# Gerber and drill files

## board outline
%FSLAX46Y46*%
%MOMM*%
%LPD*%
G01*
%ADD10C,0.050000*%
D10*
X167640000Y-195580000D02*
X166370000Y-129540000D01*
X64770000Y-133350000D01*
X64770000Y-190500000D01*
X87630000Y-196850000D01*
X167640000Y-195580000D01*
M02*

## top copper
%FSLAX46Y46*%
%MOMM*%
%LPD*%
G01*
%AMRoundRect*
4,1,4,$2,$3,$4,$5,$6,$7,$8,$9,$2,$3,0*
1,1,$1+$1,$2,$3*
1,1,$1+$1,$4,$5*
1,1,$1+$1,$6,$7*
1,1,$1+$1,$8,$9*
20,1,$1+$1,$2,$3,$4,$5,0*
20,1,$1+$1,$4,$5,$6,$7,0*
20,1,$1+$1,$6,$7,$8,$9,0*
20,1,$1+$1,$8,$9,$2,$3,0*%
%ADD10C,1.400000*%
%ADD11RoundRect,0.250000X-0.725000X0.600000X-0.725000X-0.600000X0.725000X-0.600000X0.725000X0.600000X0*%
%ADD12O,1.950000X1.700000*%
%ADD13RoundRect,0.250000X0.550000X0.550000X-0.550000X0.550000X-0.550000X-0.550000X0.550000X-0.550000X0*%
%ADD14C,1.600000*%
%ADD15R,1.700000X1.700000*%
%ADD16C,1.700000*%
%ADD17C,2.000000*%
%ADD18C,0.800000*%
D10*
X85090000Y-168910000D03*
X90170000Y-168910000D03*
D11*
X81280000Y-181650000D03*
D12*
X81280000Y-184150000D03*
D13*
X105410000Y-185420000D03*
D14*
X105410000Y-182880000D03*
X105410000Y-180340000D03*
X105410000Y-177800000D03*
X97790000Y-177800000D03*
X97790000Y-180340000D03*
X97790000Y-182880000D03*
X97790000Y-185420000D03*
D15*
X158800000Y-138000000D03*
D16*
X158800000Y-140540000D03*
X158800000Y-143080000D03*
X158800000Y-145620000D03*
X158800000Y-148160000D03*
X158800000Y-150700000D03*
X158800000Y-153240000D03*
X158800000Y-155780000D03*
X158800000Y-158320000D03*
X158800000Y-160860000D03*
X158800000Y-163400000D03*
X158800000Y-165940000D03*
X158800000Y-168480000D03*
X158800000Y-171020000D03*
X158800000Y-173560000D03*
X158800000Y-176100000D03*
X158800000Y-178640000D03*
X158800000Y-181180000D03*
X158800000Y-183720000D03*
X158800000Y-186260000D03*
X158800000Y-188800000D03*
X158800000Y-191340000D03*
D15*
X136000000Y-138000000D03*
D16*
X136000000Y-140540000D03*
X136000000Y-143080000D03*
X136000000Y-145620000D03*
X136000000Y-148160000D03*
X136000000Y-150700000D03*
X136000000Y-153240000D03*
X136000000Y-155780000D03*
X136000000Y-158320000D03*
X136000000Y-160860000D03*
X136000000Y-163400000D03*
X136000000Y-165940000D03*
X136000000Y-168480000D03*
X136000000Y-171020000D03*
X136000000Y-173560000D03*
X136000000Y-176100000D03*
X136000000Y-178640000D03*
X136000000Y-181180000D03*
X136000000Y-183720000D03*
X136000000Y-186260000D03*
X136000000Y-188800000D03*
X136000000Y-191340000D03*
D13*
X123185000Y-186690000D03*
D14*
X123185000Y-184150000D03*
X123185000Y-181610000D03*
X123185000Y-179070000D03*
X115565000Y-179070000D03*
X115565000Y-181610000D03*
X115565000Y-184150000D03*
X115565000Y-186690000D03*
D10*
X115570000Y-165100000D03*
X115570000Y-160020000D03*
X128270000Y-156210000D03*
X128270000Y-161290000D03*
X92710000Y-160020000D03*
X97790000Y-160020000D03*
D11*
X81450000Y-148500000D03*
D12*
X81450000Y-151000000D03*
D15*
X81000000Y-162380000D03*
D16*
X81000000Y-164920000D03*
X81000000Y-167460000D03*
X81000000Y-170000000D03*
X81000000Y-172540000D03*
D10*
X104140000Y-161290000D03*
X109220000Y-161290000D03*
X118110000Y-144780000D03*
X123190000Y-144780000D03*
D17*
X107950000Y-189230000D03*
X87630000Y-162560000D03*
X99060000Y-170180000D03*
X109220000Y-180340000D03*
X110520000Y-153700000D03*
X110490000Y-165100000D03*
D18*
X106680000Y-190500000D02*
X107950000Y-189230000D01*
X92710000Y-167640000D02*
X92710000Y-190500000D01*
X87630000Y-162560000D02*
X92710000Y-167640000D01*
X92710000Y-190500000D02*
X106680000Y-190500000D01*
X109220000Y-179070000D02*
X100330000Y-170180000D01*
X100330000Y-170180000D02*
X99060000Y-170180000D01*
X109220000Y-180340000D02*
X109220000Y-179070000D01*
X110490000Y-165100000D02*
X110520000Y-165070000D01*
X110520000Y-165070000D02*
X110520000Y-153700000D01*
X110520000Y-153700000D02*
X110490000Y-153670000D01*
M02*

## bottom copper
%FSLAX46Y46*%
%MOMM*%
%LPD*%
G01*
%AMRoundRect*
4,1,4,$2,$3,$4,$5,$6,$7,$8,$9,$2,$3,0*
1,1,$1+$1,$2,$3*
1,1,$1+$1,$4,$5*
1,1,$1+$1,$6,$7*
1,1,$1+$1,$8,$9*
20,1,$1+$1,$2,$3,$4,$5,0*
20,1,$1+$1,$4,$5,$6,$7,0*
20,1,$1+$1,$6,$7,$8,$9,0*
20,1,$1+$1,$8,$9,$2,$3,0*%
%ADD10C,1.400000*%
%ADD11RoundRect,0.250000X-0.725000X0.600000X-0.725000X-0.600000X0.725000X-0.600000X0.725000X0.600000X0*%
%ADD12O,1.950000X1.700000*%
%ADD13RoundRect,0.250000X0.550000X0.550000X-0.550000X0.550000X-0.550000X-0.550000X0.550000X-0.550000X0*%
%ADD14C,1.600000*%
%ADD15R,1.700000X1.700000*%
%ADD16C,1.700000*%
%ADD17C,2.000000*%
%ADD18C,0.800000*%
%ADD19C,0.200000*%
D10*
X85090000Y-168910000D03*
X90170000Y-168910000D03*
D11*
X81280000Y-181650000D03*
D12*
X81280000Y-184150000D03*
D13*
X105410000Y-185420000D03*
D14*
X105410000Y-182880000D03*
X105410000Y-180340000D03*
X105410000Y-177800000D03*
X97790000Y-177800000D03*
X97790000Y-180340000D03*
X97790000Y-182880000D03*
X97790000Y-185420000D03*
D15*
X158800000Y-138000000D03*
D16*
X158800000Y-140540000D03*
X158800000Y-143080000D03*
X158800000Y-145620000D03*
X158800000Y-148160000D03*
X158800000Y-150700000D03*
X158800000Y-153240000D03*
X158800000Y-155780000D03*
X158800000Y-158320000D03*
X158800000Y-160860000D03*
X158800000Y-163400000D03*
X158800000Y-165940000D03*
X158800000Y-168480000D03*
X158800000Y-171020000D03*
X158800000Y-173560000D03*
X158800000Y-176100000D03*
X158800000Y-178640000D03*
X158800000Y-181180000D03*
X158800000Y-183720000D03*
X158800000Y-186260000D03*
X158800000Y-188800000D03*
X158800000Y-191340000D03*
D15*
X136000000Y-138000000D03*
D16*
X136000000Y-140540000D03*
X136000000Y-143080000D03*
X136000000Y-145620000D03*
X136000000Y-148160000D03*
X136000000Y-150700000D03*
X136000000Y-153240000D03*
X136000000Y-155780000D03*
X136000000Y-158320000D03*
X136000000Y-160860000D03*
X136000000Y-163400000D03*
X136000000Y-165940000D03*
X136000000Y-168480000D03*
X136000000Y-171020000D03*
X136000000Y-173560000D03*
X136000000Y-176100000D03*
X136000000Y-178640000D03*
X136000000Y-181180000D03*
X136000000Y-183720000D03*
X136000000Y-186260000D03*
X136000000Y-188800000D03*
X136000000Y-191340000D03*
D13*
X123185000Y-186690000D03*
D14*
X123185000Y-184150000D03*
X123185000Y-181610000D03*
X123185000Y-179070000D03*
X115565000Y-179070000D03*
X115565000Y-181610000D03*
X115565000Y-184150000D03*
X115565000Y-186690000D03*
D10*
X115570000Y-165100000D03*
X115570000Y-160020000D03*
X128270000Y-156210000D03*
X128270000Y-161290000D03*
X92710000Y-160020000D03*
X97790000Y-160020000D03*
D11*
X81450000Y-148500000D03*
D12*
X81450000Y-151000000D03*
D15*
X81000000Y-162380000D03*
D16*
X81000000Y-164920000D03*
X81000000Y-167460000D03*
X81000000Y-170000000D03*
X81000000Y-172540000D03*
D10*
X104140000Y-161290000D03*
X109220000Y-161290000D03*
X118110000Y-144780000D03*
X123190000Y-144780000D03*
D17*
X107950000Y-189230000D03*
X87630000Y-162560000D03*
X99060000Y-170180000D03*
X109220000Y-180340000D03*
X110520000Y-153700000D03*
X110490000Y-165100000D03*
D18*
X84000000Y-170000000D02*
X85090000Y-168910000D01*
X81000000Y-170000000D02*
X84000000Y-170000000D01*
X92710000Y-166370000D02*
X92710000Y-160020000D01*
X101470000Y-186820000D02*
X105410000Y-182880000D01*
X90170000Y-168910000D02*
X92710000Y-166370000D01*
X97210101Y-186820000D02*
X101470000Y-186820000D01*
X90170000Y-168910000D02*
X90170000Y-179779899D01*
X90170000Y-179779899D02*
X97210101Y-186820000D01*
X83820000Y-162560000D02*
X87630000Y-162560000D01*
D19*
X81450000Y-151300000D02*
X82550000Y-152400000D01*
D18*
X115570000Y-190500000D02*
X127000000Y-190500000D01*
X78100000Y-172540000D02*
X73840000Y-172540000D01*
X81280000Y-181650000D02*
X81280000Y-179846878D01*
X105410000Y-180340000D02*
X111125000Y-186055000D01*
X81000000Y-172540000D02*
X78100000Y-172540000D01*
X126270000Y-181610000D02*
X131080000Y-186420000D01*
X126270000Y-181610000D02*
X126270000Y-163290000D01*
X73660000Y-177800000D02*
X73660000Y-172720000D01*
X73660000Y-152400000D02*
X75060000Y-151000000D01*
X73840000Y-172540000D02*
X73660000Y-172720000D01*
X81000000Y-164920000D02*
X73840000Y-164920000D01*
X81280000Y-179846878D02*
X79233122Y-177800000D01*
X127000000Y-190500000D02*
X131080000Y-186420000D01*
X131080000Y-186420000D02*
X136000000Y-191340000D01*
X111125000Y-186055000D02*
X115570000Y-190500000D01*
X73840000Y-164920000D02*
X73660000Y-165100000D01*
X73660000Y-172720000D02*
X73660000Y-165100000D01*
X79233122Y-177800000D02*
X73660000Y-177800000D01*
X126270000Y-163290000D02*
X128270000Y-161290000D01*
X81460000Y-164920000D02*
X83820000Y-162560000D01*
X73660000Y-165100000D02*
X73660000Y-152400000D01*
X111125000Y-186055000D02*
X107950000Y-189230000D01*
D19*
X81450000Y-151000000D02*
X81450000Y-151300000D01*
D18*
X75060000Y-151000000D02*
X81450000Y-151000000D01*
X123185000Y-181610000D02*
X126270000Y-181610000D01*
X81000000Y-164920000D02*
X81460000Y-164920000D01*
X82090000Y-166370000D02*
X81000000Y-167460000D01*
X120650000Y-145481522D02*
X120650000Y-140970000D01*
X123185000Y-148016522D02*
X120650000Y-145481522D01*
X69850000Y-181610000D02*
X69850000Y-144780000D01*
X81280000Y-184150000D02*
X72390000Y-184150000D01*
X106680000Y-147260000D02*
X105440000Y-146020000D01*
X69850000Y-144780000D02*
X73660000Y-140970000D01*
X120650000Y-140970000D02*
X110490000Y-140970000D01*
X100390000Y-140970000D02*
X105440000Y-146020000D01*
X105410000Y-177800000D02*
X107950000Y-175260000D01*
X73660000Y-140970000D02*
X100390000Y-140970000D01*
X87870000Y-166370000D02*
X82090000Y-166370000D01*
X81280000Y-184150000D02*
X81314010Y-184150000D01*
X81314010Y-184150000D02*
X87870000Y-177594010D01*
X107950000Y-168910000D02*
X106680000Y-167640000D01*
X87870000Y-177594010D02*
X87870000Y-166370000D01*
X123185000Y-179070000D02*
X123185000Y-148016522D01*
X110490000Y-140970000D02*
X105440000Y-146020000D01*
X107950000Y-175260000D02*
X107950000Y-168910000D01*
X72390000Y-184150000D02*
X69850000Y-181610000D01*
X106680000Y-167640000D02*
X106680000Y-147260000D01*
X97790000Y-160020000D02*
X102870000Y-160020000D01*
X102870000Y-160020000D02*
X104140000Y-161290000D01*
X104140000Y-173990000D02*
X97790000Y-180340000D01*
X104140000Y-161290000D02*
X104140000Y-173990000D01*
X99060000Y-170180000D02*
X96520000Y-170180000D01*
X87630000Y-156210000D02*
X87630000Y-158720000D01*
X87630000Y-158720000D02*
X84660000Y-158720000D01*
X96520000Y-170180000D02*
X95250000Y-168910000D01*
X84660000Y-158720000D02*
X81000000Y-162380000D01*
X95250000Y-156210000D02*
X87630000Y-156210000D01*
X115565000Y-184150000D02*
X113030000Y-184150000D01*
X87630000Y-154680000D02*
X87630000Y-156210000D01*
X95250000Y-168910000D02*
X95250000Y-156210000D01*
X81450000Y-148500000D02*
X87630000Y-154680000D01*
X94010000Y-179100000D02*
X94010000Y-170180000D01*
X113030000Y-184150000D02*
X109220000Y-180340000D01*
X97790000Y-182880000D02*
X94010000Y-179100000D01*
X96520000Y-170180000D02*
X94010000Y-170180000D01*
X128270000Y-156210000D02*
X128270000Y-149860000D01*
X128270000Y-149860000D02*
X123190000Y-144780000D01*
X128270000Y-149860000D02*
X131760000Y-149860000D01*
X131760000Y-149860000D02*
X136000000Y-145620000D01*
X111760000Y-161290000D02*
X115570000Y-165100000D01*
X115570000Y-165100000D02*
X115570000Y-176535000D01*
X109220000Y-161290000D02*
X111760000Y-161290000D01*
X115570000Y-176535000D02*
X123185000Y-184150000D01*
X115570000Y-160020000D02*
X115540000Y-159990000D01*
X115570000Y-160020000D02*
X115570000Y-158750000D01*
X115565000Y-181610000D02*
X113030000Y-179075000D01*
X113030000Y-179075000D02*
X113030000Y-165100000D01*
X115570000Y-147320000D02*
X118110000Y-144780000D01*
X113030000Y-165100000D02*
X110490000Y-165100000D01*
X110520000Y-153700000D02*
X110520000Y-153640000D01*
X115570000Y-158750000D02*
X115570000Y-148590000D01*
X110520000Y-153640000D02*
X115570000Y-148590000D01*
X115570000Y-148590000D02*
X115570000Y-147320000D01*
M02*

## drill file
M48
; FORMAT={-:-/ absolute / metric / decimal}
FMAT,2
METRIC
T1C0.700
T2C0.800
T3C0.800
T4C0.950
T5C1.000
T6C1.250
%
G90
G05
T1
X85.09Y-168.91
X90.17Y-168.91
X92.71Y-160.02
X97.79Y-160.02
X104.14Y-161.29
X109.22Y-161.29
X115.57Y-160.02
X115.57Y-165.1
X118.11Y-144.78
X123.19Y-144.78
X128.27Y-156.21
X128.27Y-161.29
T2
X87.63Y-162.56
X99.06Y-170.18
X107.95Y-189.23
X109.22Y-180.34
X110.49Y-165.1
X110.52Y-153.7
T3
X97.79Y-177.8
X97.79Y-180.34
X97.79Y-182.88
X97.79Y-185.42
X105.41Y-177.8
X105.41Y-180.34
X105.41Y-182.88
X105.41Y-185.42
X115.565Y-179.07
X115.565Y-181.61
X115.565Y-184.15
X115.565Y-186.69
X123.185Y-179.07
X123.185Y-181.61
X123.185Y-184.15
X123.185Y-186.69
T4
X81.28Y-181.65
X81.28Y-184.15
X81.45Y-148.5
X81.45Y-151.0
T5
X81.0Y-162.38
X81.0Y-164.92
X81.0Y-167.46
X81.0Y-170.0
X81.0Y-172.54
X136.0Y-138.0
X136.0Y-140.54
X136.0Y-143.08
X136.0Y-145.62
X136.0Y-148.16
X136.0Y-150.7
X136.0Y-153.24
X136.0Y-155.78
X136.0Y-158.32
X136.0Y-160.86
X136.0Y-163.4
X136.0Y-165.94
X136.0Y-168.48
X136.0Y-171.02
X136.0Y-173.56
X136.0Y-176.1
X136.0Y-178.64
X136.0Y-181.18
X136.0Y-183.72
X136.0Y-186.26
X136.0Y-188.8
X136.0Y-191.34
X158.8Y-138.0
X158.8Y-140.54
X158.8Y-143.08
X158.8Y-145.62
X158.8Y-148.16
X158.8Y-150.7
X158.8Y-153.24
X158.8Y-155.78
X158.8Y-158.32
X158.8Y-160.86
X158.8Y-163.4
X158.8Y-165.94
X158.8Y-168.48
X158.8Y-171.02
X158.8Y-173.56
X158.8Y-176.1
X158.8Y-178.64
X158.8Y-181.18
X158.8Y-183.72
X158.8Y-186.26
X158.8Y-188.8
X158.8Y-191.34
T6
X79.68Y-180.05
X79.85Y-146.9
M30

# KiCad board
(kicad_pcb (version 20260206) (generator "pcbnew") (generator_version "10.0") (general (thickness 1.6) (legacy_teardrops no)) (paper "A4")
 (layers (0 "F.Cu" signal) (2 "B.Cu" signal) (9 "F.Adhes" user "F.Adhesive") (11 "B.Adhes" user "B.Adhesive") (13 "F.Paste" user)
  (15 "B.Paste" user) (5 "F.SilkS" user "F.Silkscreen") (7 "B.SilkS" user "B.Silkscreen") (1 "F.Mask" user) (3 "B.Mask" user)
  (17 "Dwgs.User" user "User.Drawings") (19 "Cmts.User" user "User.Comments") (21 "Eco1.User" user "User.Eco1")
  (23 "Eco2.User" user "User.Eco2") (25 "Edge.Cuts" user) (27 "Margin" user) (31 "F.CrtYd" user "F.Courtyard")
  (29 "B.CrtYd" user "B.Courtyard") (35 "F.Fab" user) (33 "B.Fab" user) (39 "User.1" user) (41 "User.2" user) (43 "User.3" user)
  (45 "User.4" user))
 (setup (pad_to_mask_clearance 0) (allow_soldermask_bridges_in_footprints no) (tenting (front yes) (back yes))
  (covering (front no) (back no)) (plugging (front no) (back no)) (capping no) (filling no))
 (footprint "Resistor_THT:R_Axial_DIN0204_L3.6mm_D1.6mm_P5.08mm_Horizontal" (layer "F.Cu") (at 85.09 168.91)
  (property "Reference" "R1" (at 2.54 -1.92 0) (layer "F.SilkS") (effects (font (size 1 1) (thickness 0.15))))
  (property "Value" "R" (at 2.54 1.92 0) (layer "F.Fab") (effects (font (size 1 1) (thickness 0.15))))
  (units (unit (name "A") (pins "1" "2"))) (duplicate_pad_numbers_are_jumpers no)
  (pad "1" thru_hole circle (at 0 0) (size 1.4 1.4) (drill 0.7) (layers "*.Cu" "*.Mask") (remove_unused_layers no) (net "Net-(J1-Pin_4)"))
  (pad "2" thru_hole circle (at 5.08 0) (size 1.4 1.4) (drill 0.7) (layers "*.Cu" "*.Mask") (remove_unused_layers no) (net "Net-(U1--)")))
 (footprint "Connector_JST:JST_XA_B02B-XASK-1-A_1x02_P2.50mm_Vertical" (layer "F.Cu") (at 81.28 181.65 -90)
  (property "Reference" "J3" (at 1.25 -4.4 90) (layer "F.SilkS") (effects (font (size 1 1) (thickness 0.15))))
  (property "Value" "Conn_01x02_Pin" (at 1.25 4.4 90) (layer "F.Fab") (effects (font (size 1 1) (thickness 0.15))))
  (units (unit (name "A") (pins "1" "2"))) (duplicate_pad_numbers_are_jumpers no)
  (pad "" np_thru_hole circle (at -1.6 1.6 270) (size 1.25 1.25) (drill 1.25) (layers "*.Cu" "*.Mask"))
  (pad "1" thru_hole roundrect (at 0 0 270) (size 1.7 1.95) (drill 0.95) (layers "*.Cu" "*.Mask") (remove_unused_layers no)
   (roundrect_rratio 0.147059) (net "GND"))
  (pad "2" thru_hole oval (at 2.5 0 270) (size 1.7 1.95) (drill 0.95) (layers "*.Cu" "*.Mask") (remove_unused_layers no) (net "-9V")))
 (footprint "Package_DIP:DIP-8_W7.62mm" (layer "F.Cu") (at 105.41 185.42 180)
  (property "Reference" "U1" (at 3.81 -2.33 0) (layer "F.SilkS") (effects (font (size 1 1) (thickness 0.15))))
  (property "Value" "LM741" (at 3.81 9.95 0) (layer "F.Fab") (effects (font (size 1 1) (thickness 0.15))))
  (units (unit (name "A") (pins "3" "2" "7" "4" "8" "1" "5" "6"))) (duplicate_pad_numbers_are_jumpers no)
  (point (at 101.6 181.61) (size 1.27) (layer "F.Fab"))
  (pad "1" thru_hole roundrect (at 0 0 180) (size 1.6 1.6) (drill 0.8) (layers "*.Cu" "*.Mask") (remove_unused_layers no)
   (roundrect_rratio 0.15625) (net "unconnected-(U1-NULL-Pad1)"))
  (pad "2" thru_hole circle (at 0 2.54 180) (size 1.6 1.6) (drill 0.8) (layers "*.Cu" "*.Mask") (remove_unused_layers no) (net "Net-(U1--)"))
  (pad "3" thru_hole circle (at 0 5.08 180) (size 1.6 1.6) (drill 0.8) (layers "*.Cu" "*.Mask") (remove_unused_layers no) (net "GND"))
  (pad "4" thru_hole circle (at 0 7.62 180) (size 1.6 1.6) (drill 0.8) (layers "*.Cu" "*.Mask") (remove_unused_layers no) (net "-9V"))
  (pad "5" thru_hole circle (at 7.62 7.62 180) (size 1.6 1.6) (drill 0.8) (layers "*.Cu" "*.Mask") (remove_unused_layers no)
   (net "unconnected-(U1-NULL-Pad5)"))
  (pad "6" thru_hole circle (at 7.62 5.08 180) (size 1.6 1.6) (drill 0.8) (layers "*.Cu" "*.Mask") (remove_unused_layers no)
   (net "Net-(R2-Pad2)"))
  (pad "7" thru_hole circle (at 7.62 2.54 180) (size 1.6 1.6) (drill 0.8) (layers "*.Cu" "*.Mask") (remove_unused_layers no) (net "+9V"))
  (pad "8" thru_hole circle (at 7.62 0 180) (size 1.6 1.6) (drill 0.8) (layers "*.Cu" "*.Mask") (remove_unused_layers no)
   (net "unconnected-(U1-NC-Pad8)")))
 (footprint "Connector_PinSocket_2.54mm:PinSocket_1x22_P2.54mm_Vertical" (layer "F.Cu") (at 158.8 138)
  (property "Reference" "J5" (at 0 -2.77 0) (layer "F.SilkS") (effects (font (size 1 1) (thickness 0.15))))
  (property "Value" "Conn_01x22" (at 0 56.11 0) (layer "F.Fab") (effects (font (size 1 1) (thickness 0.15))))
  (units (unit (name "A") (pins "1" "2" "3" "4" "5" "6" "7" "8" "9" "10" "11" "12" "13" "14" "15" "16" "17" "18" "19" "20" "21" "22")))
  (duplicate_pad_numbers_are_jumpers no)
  (pad "1" thru_hole rect (at 0 0) (size 1.7 1.7) (drill 1) (layers "*.Cu" "*.Mask") (remove_unused_layers no)
   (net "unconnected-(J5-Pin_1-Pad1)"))
  (pad "2" thru_hole circle (at 0 2.54) (size 1.7 1.7) (drill 1) (layers "*.Cu" "*.Mask") (remove_unused_layers no)
   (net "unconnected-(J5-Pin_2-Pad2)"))
  (pad "3" thru_hole circle (at 0 5.08) (size 1.7 1.7) (drill 1) (layers "*.Cu" "*.Mask") (remove_unused_layers no)
   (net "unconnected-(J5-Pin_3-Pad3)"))
  (pad "4" thru_hole circle (at 0 7.62) (size 1.7 1.7) (drill 1) (layers "*.Cu" "*.Mask") (remove_unused_layers no)
   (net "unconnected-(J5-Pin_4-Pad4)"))
  (pad "5" thru_hole circle (at 0 10.16) (size 1.7 1.7) (drill 1) (layers "*.Cu" "*.Mask") (remove_unused_layers no)
   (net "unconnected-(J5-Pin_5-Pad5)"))
  (pad "6" thru_hole circle (at 0 12.7) (size 1.7 1.7) (drill 1) (layers "*.Cu" "*.Mask") (remove_unused_layers no)
   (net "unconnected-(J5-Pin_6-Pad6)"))
  (pad "7" thru_hole circle (at 0 15.24) (size 1.7 1.7) (drill 1) (layers "*.Cu" "*.Mask") (remove_unused_layers no)
   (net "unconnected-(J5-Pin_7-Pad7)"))
  (pad "8" thru_hole circle (at 0 17.78) (size 1.7 1.7) (drill 1) (layers "*.Cu" "*.Mask") (remove_unused_layers no)
   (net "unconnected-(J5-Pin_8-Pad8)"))
  (pad "9" thru_hole circle (at 0 20.32) (size 1.7 1.7) (drill 1) (layers "*.Cu" "*.Mask") (remove_unused_layers no)
   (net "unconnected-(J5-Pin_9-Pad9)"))
  (pad "10" thru_hole circle (at 0 22.86) (size 1.7 1.7) (drill 1) (layers "*.Cu" "*.Mask") (remove_unused_layers no)
   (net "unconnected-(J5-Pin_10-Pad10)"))
  (pad "11" thru_hole circle (at 0 25.4) (size 1.7 1.7) (drill 1) (layers "*.Cu" "*.Mask") (remove_unused_layers no)
   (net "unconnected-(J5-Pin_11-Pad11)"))
  (pad "12" thru_hole circle (at 0 27.94) (size 1.7 1.7) (drill 1) (layers "*.Cu" "*.Mask") (remove_unused_layers no)
   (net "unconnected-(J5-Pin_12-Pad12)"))
  (pad "13" thru_hole circle (at 0 30.48) (size 1.7 1.7) (drill 1) (layers "*.Cu" "*.Mask") (remove_unused_layers no)
   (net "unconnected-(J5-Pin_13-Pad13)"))
  (pad "14" thru_hole circle (at 0 33.02) (size 1.7 1.7) (drill 1) (layers "*.Cu" "*.Mask") (remove_unused_layers no)
   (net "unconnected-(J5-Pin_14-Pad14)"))
  (pad "15" thru_hole circle (at 0 35.56) (size 1.7 1.7) (drill 1) (layers "*.Cu" "*.Mask") (remove_unused_layers no)
   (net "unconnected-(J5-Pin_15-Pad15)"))
  (pad "16" thru_hole circle (at 0 38.1) (size 1.7 1.7) (drill 1) (layers "*.Cu" "*.Mask") (remove_unused_layers no)
   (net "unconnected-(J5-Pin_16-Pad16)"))
  (pad "17" thru_hole circle (at 0 40.64) (size 1.7 1.7) (drill 1) (layers "*.Cu" "*.Mask") (remove_unused_layers no)
   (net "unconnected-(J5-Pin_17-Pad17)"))
  (pad "18" thru_hole circle (at 0 43.18) (size 1.7 1.7) (drill 1) (layers "*.Cu" "*.Mask") (remove_unused_layers no)
   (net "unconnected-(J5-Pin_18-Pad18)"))
  (pad "19" thru_hole circle (at 0 45.72) (size 1.7 1.7) (drill 1) (layers "*.Cu" "*.Mask") (remove_unused_layers no)
   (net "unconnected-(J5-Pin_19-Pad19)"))
  (pad "20" thru_hole circle (at 0 48.26) (size 1.7 1.7) (drill 1) (layers "*.Cu" "*.Mask") (remove_unused_layers no)
   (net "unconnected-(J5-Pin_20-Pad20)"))
  (pad "21" thru_hole circle (at 0 50.8) (size 1.7 1.7) (drill 1) (layers "*.Cu" "*.Mask") (remove_unused_layers no)
   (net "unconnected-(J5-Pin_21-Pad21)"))
  (pad "22" thru_hole circle (at 0 53.34) (size 1.7 1.7) (drill 1) (layers "*.Cu" "*.Mask") (remove_unused_layers no)
   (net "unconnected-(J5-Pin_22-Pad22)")))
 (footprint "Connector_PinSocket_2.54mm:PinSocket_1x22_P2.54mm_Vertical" (layer "F.Cu") (at 136 138)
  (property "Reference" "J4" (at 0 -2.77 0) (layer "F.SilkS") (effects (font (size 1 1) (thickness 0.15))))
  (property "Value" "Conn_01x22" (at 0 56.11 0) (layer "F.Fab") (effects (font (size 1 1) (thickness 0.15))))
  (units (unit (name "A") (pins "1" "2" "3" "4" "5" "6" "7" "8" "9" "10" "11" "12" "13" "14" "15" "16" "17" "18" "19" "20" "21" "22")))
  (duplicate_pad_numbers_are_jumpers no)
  (pad "1" thru_hole rect (at 0 0) (size 1.7 1.7) (drill 1) (layers "*.Cu" "*.Mask") (remove_unused_layers no)
   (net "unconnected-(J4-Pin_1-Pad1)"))
  (pad "2" thru_hole circle (at 0 2.54) (size 1.7 1.7) (drill 1) (layers "*.Cu" "*.Mask") (remove_unused_layers no)
   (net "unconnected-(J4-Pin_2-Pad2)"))
  (pad "3" thru_hole circle (at 0 5.08) (size 1.7 1.7) (drill 1) (layers "*.Cu" "*.Mask") (remove_unused_layers no)
   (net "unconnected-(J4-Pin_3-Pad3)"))
  (pad "4" thru_hole circle (at 0 7.62) (size 1.7 1.7) (drill 1) (layers "*.Cu" "*.Mask") (remove_unused_layers no) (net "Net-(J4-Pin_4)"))
  (pad "5" thru_hole circle (at 0 10.16) (size 1.7 1.7) (drill 1) (layers "*.Cu" "*.Mask") (remove_unused_layers no)
   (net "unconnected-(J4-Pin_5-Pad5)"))
  (pad "6" thru_hole circle (at 0 12.7) (size 1.7 1.7) (drill 1) (layers "*.Cu" "*.Mask") (remove_unused_layers no)
   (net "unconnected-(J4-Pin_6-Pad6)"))
  (pad "7" thru_hole circle (at 0 15.24) (size 1.7 1.7) (drill 1) (layers "*.Cu" "*.Mask") (remove_unused_layers no)
   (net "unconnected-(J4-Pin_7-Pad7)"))
  (pad "8" thru_hole circle (at 0 17.78) (size 1.7 1.7) (drill 1) (layers "*.Cu" "*.Mask") (remove_unused_layers no)
   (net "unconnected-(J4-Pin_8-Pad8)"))
  (pad "9" thru_hole circle (at 0 20.32) (size 1.7 1.7) (drill 1) (layers "*.Cu" "*.Mask") (remove_unused_layers no)
   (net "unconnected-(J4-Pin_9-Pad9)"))
  (pad "10" thru_hole circle (at 0 22.86) (size 1.7 1.7) (drill 1) (layers "*.Cu" "*.Mask") (remove_unused_layers no)
   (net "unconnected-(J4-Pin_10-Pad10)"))
  (pad "11" thru_hole circle (at 0 25.4) (size 1.7 1.7) (drill 1) (layers "*.Cu" "*.Mask") (remove_unused_layers no)
   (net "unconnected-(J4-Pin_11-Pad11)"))
  (pad "12" thru_hole circle (at 0 27.94) (size 1.7 1.7) (drill 1) (layers "*.Cu" "*.Mask") (remove_unused_layers no)
   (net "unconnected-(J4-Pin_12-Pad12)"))
  (pad "13" thru_hole circle (at 0 30.48) (size 1.7 1.7) (drill 1) (layers "*.Cu" "*.Mask") (remove_unused_layers no)
   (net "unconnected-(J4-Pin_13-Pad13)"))
  (pad "14" thru_hole circle (at 0 33.02) (size 1.7 1.7) (drill 1) (layers "*.Cu" "*.Mask") (remove_unused_layers no)
   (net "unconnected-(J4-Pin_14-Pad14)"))
  (pad "15" thru_hole circle (at 0 35.56) (size 1.7 1.7) (drill 1) (layers "*.Cu" "*.Mask") (remove_unused_layers no)
   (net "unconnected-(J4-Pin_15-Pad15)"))
  (pad "16" thru_hole circle (at 0 38.1) (size 1.7 1.7) (drill 1) (layers "*.Cu" "*.Mask") (remove_unused_layers no)
   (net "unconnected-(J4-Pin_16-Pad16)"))
  (pad "17" thru_hole circle (at 0 40.64) (size 1.7 1.7) (drill 1) (layers "*.Cu" "*.Mask") (remove_unused_layers no)
   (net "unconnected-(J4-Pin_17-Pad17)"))
  (pad "18" thru_hole circle (at 0 43.18) (size 1.7 1.7) (drill 1) (layers "*.Cu" "*.Mask") (remove_unused_layers no)
   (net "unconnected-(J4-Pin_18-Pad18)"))
  (pad "19" thru_hole circle (at 0 45.72) (size 1.7 1.7) (drill 1) (layers "*.Cu" "*.Mask") (remove_unused_layers no)
   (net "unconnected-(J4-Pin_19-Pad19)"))
  (pad "20" thru_hole circle (at 0 48.26) (size 1.7 1.7) (drill 1) (layers "*.Cu" "*.Mask") (remove_unused_layers no)
   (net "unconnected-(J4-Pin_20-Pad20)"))
  (pad "21" thru_hole circle (at 0 50.8) (size 1.7 1.7) (drill 1) (layers "*.Cu" "*.Mask") (remove_unused_layers no)
   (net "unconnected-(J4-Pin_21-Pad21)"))
  (pad "22" thru_hole circle (at 0 53.34) (size 1.7 1.7) (drill 1) (layers "*.Cu" "*.Mask") (remove_unused_layers no) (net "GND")))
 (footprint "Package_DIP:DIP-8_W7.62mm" (layer "F.Cu") (at 123.185 186.69 180)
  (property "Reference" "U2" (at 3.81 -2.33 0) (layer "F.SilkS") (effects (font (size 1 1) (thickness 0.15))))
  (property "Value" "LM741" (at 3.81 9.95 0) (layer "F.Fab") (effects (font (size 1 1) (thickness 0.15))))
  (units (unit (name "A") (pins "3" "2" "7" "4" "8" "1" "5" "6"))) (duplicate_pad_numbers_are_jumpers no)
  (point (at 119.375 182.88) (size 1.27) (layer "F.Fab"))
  (pad "1" thru_hole roundrect (at 0 0 180) (size 1.6 1.6) (drill 0.8) (layers "*.Cu" "*.Mask") (remove_unused_layers no)
   (roundrect_rratio 0.15625) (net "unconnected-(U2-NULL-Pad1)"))
  (pad "2" thru_hole circle (at 0 2.54 180) (size 1.6 1.6) (drill 0.8) (layers "*.Cu" "*.Mask") (remove_unused_layers no) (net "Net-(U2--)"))
  (pad "3" thru_hole circle (at 0 5.08 180) (size 1.6 1.6) (drill 0.8) (layers "*.Cu" "*.Mask") (remove_unused_layers no) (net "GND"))
  (pad "4" thru_hole circle (at 0 7.62 180) (size 1.6 1.6) (drill 0.8) (layers "*.Cu" "*.Mask") (remove_unused_layers no) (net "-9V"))
  (pad "5" thru_hole circle (at 7.62 7.62 180) (size 1.6 1.6) (drill 0.8) (layers "*.Cu" "*.Mask") (remove_unused_layers no)
   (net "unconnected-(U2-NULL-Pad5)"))
  (pad "6" thru_hole circle (at 7.62 5.08 180) (size 1.6 1.6) (drill 0.8) (layers "*.Cu" "*.Mask") (remove_unused_layers no)
   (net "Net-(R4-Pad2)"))
  (pad "7" thru_hole circle (at 7.62 2.54 180) (size 1.6 1.6) (drill 0.8) (layers "*.Cu" "*.Mask") (remove_unused_layers no) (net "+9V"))
  (pad "8" thru_hole circle (at 7.62 0 180) (size 1.6 1.6) (drill 0.8) (layers "*.Cu" "*.Mask") (remove_unused_layers no)
   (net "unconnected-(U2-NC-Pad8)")))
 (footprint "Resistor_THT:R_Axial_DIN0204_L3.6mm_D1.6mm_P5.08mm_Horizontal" (layer "F.Cu") (at 115.57 165.1 90)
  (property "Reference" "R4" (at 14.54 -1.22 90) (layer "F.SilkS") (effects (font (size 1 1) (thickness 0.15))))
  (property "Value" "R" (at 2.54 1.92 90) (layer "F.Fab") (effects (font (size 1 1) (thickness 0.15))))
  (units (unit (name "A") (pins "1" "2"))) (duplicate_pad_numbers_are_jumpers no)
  (pad "1" thru_hole circle (at 0 0 90) (size 1.4 1.4) (drill 0.7) (layers "*.Cu" "*.Mask") (remove_unused_layers no) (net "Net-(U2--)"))
  (pad "2" thru_hole circle (at 5.08 0 90) (size 1.4 1.4) (drill 0.7) (layers "*.Cu" "*.Mask") (remove_unused_layers no)
   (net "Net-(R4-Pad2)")))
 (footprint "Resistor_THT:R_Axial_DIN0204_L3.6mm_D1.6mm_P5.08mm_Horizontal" (layer "F.Cu") (at 128.27 156.21 -90)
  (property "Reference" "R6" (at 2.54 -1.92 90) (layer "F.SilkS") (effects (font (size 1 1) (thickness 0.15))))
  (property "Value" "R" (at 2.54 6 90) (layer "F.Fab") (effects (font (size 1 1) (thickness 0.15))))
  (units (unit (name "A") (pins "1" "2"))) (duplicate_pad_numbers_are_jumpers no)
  (pad "1" thru_hole circle (at 0 0 270) (size 1.4 1.4) (drill 0.7) (layers "*.Cu" "*.Mask") (remove_unused_layers no)
   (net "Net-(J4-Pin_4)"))
  (pad "2" thru_hole circle (at 5.08 0 270) (size 1.4 1.4) (drill 0.7) (layers "*.Cu" "*.Mask") (remove_unused_layers no) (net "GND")))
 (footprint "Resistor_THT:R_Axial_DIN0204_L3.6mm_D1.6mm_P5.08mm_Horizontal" (layer "F.Cu") (at 92.71 160.02)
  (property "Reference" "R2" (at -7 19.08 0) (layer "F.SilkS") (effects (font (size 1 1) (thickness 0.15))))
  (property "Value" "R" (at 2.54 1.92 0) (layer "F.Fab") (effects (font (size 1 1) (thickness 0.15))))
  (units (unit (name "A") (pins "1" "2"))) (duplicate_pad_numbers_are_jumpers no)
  (pad "1" thru_hole circle (at 0 0) (size 1.4 1.4) (drill 0.7) (layers "*.Cu" "*.Mask") (remove_unused_layers no) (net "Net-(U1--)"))
  (pad "2" thru_hole circle (at 5.08 0) (size 1.4 1.4) (drill 0.7) (layers "*.Cu" "*.Mask") (remove_unused_layers no) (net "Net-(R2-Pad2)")))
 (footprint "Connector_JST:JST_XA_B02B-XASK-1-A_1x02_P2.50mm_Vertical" (layer "F.Cu") (at 81.45 148.5 -90)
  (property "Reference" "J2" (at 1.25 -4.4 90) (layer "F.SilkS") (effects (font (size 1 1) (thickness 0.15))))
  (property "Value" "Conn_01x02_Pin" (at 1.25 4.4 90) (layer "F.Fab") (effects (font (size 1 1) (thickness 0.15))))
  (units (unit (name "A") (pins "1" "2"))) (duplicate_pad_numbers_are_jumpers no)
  (pad "" np_thru_hole circle (at -1.6 1.6 270) (size 1.25 1.25) (drill 1.25) (layers "*.Cu" "*.Mask"))
  (pad "1" thru_hole roundrect (at 0 0 270) (size 1.7 1.95) (drill 0.95) (layers "*.Cu" "*.Mask") (remove_unused_layers no)
   (roundrect_rratio 0.147059) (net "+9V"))
  (pad "2" thru_hole oval (at 2.5 0 270) (size 1.7 1.95) (drill 0.95) (layers "*.Cu" "*.Mask") (remove_unused_layers no) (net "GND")))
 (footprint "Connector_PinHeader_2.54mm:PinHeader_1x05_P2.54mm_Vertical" (layer "F.Cu") (at 81 162.38)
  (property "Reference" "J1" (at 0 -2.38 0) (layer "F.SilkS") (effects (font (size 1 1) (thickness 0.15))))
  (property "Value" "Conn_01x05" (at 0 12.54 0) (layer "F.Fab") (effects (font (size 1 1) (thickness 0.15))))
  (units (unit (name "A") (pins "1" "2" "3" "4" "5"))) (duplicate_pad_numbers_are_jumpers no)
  (pad "1" thru_hole rect (at 0 0) (size 1.7 1.7) (drill 1) (layers "*.Cu" "*.Mask") (remove_unused_layers no) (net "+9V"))
  (pad "2" thru_hole circle (at 0 2.54) (size 1.7 1.7) (drill 1) (layers "*.Cu" "*.Mask") (remove_unused_layers no) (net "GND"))
  (pad "3" thru_hole circle (at 0 5.08) (size 1.7 1.7) (drill 1) (layers "*.Cu" "*.Mask") (remove_unused_layers no) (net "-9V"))
  (pad "4" thru_hole circle (at 0 7.62) (size 1.7 1.7) (drill 1) (layers "*.Cu" "*.Mask") (remove_unused_layers no) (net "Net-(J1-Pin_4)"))
  (pad "5" thru_hole circle (at 0 10.16) (size 1.7 1.7) (drill 1) (layers "*.Cu" "*.Mask") (remove_unused_layers no) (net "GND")))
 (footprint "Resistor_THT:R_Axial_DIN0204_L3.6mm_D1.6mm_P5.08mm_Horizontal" (layer "F.Cu") (at 104.14 161.29)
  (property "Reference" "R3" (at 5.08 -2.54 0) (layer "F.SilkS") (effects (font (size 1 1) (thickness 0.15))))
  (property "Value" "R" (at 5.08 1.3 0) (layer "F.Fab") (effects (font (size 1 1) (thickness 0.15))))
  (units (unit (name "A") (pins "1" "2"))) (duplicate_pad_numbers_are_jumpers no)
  (pad "1" thru_hole circle (at 0 0) (size 1.4 1.4) (drill 0.7) (layers "*.Cu" "*.Mask") (remove_unused_layers no) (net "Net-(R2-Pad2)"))
  (pad "2" thru_hole circle (at 5.08 0) (size 1.4 1.4) (drill 0.7) (layers "*.Cu" "*.Mask") (remove_unused_layers no) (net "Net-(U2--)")))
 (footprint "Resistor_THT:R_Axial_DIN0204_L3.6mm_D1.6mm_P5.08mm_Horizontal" (layer "F.Cu") (at 118.11 144.78)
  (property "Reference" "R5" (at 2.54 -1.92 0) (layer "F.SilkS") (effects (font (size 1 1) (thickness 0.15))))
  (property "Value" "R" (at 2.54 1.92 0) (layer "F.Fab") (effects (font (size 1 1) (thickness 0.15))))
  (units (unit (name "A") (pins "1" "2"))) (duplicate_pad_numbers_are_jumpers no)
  (pad "1" thru_hole circle (at 0 0) (size 1.4 1.4) (drill 0.7) (layers "*.Cu" "*.Mask") (remove_unused_layers no) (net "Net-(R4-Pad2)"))
  (pad "2" thru_hole circle (at 5.08 0) (size 1.4 1.4) (drill 0.7) (layers "*.Cu" "*.Mask") (remove_unused_layers no) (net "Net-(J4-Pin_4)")))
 (gr_poly
  (pts (xy 167.64 195.58) (xy 166.37 129.54) (xy 64.77 133.35) (xy 64.77 190.5) (xy 87.63 196.85)) (stroke (width 0.05) (type solid))
  (fill no) (layer "Edge.Cuts"))
 (segment (start 84 170) (end 85.09 168.91) (width 0.8) (layer "B.Cu") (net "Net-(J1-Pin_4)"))
 (segment (start 81 170) (end 84 170) (width 0.8) (layer "B.Cu") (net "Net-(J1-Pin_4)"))
 (segment (start 92.71 166.37) (end 92.71 160.02) (width 0.8) (layer "B.Cu") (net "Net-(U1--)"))
 (segment (start 101.47 186.82) (end 105.41 182.88) (width 0.8) (layer "B.Cu") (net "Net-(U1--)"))
 (segment (start 90.17 168.91) (end 92.71 166.37) (width 0.8) (layer "B.Cu") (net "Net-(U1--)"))
 (segment (start 97.210101 186.82) (end 101.47 186.82) (width 0.8) (layer "B.Cu") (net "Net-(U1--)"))
 (segment (start 90.17 168.91) (end 90.17 179.779899) (width 0.8) (layer "B.Cu") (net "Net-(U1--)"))
 (segment (start 90.17 179.779899) (end 97.210101 186.82) (width 0.8) (layer "B.Cu") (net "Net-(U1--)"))
 (segment (start 106.68 190.5) (end 107.95 189.23) (width 0.8) (layer "F.Cu") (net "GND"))
 (segment (start 92.71 167.64) (end 92.71 190.5) (width 0.8) (layer "F.Cu") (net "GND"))
 (segment (start 87.63 162.56) (end 92.71 167.64) (width 0.8) (layer "F.Cu") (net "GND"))
 (segment (start 92.71 190.5) (end 106.68 190.5) (width 0.8) (layer "F.Cu") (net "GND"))
 (via (at 107.95 189.23) (size 2) (drill 0.8) (layers "F.Cu" "B.Cu") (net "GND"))
 (via (at 87.63 162.56) (size 2) (drill 0.8) (layers "F.Cu" "B.Cu") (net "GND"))
 (segment (start 83.82 162.56) (end 87.63 162.56) (width 0.8) (layer "B.Cu") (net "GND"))
 (segment (start 81.45 151.3) (end 82.55 152.4) (width 0.2) (layer "B.Cu") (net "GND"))
 (segment (start 115.57 190.5) (end 127 190.5) (width 0.8) (layer "B.Cu") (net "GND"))
 (segment (start 78.1 172.54) (end 73.84 172.54) (width 0.8) (layer "B.Cu") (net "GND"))
 (segment (start 81.28 181.65) (end 81.28 179.846878) (width 0.8) (layer "B.Cu") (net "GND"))
 (segment (start 105.41 180.34) (end 111.125 186.055) (width 0.8) (layer "B.Cu") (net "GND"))
 (segment (start 81 172.54) (end 78.1 172.54) (width 0.8) (layer "B.Cu") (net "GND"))
 (segment (start 126.27 181.61) (end 131.08 186.42) (width 0.8) (layer "B.Cu") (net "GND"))
 (segment (start 126.27 181.61) (end 126.27 163.29) (width 0.8) (layer "B.Cu") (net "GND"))
 (segment (start 73.66 177.8) (end 73.66 172.72) (width 0.8) (layer "B.Cu") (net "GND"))
 (segment (start 73.66 152.4) (end 75.06 151) (width 0.8) (layer "B.Cu") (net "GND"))
 (segment (start 73.84 172.54) (end 73.66 172.72) (width 0.8) (layer "B.Cu") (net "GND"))
 (segment (start 81 164.92) (end 73.84 164.92) (width 0.8) (layer "B.Cu") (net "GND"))
 (segment (start 81.28 179.846878) (end 79.233122 177.8) (width 0.8) (layer "B.Cu") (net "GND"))
 (segment (start 127 190.5) (end 131.08 186.42) (width 0.8) (layer "B.Cu") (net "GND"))
 (segment (start 131.08 186.42) (end 136 191.34) (width 0.8) (layer "B.Cu") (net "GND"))
 (segment (start 111.125 186.055) (end 115.57 190.5) (width 0.8) (layer "B.Cu") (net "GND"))
 (segment (start 73.84 164.92) (end 73.66 165.1) (width 0.8) (layer "B.Cu") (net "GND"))
 (segment (start 73.66 172.72) (end 73.66 165.1) (width 0.8) (layer "B.Cu") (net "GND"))
 (segment (start 79.233122 177.8) (end 73.66 177.8) (width 0.8) (layer "B.Cu") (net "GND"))
 (segment (start 126.27 163.29) (end 128.27 161.29) (width 0.8) (layer "B.Cu") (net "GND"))
 (segment (start 81.46 164.92) (end 83.82 162.56) (width 0.8) (layer "B.Cu") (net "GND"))
 (segment (start 73.66 165.1) (end 73.66 152.4) (width 0.8) (layer "B.Cu") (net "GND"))
 (segment (start 111.125 186.055) (end 107.95 189.23) (width 0.8) (layer "B.Cu") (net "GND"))
 (segment (start 81.45 151) (end 81.45 151.3) (width 0.2) (layer "B.Cu") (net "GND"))
 (segment (start 75.06 151) (end 81.45 151) (width 0.8) (layer "B.Cu") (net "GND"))
 (segment (start 123.185 181.61) (end 126.27 181.61) (width 0.8) (layer "B.Cu") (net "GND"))
 (segment (start 81 164.92) (end 81.46 164.92) (width 0.8) (layer "B.Cu") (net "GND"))
 (segment (start 82.09 166.37) (end 81 167.46) (width 0.8) (layer "B.Cu") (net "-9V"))
 (segment (start 120.65 145.481522) (end 120.65 140.97) (width 0.8) (layer "B.Cu") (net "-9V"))
 (segment (start 123.185 148.016522) (end 120.65 145.481522) (width 0.8) (layer "B.Cu") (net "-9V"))
 (segment (start 69.85 181.61) (end 69.85 144.78) (width 0.8) (layer "B.Cu") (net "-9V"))
 (segment (start 81.28 184.15) (end 72.39 184.15) (width 0.8) (layer "B.Cu") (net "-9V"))
 (segment (start 106.68 147.26) (end 105.44 146.02) (width 0.8) (layer "B.Cu") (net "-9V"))
 (segment (start 69.85 144.78) (end 73.66 140.97) (width 0.8) (layer "B.Cu") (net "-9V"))
 (segment (start 120.65 140.97) (end 110.49 140.97) (width 0.8) (layer "B.Cu") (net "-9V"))
 (segment (start 100.39 140.97) (end 105.44 146.02) (width 0.8) (layer "B.Cu") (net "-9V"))
 (segment (start 105.41 177.8) (end 107.95 175.26) (width 0.8) (layer "B.Cu") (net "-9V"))
 (segment (start 73.66 140.97) (end 100.39 140.97) (width 0.8) (layer "B.Cu") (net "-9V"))
 (segment (start 87.87 166.37) (end 82.09 166.37) (width 0.8) (layer "B.Cu") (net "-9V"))
 (segment (start 81.28 184.15) (end 81.31401 184.15) (width 0.8) (layer "B.Cu") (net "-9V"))
 (segment (start 81.31401 184.15) (end 87.87 177.59401) (width 0.8) (layer "B.Cu") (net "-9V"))
 (segment (start 107.95 168.91) (end 106.68 167.64) (width 0.8) (layer "B.Cu") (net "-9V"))
 (segment (start 87.87 177.59401) (end 87.87 166.37) (width 0.8) (layer "B.Cu") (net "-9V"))
 (segment (start 123.185 179.07) (end 123.185 148.016522) (width 0.8) (layer "B.Cu") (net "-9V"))
 (segment (start 110.49 140.97) (end 105.44 146.02) (width 0.8) (layer "B.Cu") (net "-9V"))
 (segment (start 107.95 175.26) (end 107.95 168.91) (width 0.8) (layer "B.Cu") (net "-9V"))
 (segment (start 72.39 184.15) (end 69.85 181.61) (width 0.8) (layer "B.Cu") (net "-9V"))
 (segment (start 106.68 167.64) (end 106.68 147.26) (width 0.8) (layer "B.Cu") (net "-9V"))
 (segment (start 97.79 160.02) (end 102.87 160.02) (width 0.8) (layer "B.Cu") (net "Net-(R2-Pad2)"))
 (segment (start 102.87 160.02) (end 104.14 161.29) (width 0.8) (layer "B.Cu") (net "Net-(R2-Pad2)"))
 (segment (start 104.14 173.99) (end 97.79 180.34) (width 0.8) (layer "B.Cu") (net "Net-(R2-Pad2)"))
 (segment (start 104.14 161.29) (end 104.14 173.99) (width 0.8) (layer "B.Cu") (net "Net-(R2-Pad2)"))
 (segment (start 109.22 179.07) (end 100.33 170.18) (width 0.8) (layer "F.Cu") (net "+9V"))
 (segment (start 100.33 170.18) (end 99.06 170.18) (width 0.8) (layer "F.Cu") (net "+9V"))
 (segment (start 109.22 180.34) (end 109.22 179.07) (width 0.8) (layer "F.Cu") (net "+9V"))
 (via (at 99.06 170.18) (size 2) (drill 0.8) (layers "F.Cu" "B.Cu") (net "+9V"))
 (via (at 109.22 180.34) (size 2) (drill 0.8) (layers "F.Cu" "B.Cu") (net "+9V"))
 (segment (start 99.06 170.18) (end 96.52 170.18) (width 0.8) (layer "B.Cu") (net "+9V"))
 (segment (start 87.63 156.21) (end 87.63 158.72) (width 0.8) (layer "B.Cu") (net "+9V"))
 (segment (start 87.63 158.72) (end 84.66 158.72) (width 0.8) (layer "B.Cu") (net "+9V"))
 (segment (start 96.52 170.18) (end 95.25 168.91) (width 0.8) (layer "B.Cu") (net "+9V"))
 (segment (start 84.66 158.72) (end 81 162.38) (width 0.8) (layer "B.Cu") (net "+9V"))
 (segment (start 95.25 156.21) (end 87.63 156.21) (width 0.8) (layer "B.Cu") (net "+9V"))
 (segment (start 115.565 184.15) (end 113.03 184.15) (width 0.8) (layer "B.Cu") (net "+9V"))
 (segment (start 87.63 154.68) (end 87.63 156.21) (width 0.8) (layer "B.Cu") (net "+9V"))
 (segment (start 95.25 168.91) (end 95.25 156.21) (width 0.8) (layer "B.Cu") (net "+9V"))
 (segment (start 81.45 148.5) (end 87.63 154.68) (width 0.8) (layer "B.Cu") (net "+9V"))
 (segment (start 94.01 179.1) (end 94.01 170.18) (width 0.8) (layer "B.Cu") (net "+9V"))
 (segment (start 113.03 184.15) (end 109.22 180.34) (width 0.8) (layer "B.Cu") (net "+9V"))
 (segment (start 97.79 182.88) (end 94.01 179.1) (width 0.8) (layer "B.Cu") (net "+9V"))
 (segment (start 96.52 170.18) (end 94.01 170.18) (width 0.8) (layer "B.Cu") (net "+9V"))
 (segment (start 128.27 156.21) (end 128.27 149.86) (width 0.8) (layer "B.Cu") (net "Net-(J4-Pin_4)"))
 (segment (start 128.27 149.86) (end 123.19 144.78) (width 0.8) (layer "B.Cu") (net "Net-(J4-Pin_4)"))
 (segment (start 128.27 149.86) (end 131.76 149.86) (width 0.8) (layer "B.Cu") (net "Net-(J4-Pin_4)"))
 (segment (start 131.76 149.86) (end 136 145.62) (width 0.8) (layer "B.Cu") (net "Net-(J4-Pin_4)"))
 (segment (start 111.76 161.29) (end 115.57 165.1) (width 0.8) (layer "B.Cu") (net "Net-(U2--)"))
 (segment (start 115.57 165.1) (end 115.57 176.535) (width 0.8) (layer "B.Cu") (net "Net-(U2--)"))
 (segment (start 109.22 161.29) (end 111.76 161.29) (width 0.8) (layer "B.Cu") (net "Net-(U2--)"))
 (segment (start 115.57 176.535) (end 123.185 184.15) (width 0.8) (layer "B.Cu") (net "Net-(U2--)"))
 (segment (start 110.49 165.1) (end 110.52 165.07) (width 0.8) (layer "F.Cu") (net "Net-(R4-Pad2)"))
 (segment (start 110.52 165.07) (end 110.52 153.7) (width 0.8) (layer "F.Cu") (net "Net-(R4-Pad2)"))
 (segment (start 110.52 153.7) (end 110.49 153.67) (width 0.8) (layer "F.Cu") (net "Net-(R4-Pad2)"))
 (via (at 110.52 153.7) (size 2) (drill 0.8) (layers "F.Cu" "B.Cu") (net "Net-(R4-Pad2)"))
 (via (at 110.49 165.1) (size 2) (drill 0.8) (layers "F.Cu" "B.Cu") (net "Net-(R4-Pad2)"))
 (segment (start 115.57 160.02) (end 115.54 159.99) (width 0.8) (layer "B.Cu") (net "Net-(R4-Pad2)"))
 (segment (start 115.57 160.02) (end 115.57 158.75) (width 0.8) (layer "B.Cu") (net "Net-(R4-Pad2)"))
 (segment (start 115.565 181.61) (end 113.03 179.075) (width 0.8) (layer "B.Cu") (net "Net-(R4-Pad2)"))
 (segment (start 113.03 179.075) (end 113.03 165.1) (width 0.8) (layer "B.Cu") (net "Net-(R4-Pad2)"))
 (segment (start 115.57 147.32) (end 118.11 144.78) (width 0.8) (layer "B.Cu") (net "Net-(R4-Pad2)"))
 (segment (start 113.03 165.1) (end 110.49 165.1) (width 0.8) (layer "B.Cu") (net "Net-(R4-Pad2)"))
 (segment (start 110.52 153.7) (end 110.52 153.64) (width 0.8) (layer "B.Cu") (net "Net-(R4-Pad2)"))
 (segment (start 115.57 158.75) (end 115.57 148.59) (width 0.8) (layer "B.Cu") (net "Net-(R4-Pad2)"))
 (segment (start 110.52 153.64) (end 115.57 148.59) (width 0.8) (layer "B.Cu") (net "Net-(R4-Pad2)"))
 (segment (start 115.57 148.59) (end 115.57 147.32) (width 0.8) (layer "B.Cu") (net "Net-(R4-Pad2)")))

